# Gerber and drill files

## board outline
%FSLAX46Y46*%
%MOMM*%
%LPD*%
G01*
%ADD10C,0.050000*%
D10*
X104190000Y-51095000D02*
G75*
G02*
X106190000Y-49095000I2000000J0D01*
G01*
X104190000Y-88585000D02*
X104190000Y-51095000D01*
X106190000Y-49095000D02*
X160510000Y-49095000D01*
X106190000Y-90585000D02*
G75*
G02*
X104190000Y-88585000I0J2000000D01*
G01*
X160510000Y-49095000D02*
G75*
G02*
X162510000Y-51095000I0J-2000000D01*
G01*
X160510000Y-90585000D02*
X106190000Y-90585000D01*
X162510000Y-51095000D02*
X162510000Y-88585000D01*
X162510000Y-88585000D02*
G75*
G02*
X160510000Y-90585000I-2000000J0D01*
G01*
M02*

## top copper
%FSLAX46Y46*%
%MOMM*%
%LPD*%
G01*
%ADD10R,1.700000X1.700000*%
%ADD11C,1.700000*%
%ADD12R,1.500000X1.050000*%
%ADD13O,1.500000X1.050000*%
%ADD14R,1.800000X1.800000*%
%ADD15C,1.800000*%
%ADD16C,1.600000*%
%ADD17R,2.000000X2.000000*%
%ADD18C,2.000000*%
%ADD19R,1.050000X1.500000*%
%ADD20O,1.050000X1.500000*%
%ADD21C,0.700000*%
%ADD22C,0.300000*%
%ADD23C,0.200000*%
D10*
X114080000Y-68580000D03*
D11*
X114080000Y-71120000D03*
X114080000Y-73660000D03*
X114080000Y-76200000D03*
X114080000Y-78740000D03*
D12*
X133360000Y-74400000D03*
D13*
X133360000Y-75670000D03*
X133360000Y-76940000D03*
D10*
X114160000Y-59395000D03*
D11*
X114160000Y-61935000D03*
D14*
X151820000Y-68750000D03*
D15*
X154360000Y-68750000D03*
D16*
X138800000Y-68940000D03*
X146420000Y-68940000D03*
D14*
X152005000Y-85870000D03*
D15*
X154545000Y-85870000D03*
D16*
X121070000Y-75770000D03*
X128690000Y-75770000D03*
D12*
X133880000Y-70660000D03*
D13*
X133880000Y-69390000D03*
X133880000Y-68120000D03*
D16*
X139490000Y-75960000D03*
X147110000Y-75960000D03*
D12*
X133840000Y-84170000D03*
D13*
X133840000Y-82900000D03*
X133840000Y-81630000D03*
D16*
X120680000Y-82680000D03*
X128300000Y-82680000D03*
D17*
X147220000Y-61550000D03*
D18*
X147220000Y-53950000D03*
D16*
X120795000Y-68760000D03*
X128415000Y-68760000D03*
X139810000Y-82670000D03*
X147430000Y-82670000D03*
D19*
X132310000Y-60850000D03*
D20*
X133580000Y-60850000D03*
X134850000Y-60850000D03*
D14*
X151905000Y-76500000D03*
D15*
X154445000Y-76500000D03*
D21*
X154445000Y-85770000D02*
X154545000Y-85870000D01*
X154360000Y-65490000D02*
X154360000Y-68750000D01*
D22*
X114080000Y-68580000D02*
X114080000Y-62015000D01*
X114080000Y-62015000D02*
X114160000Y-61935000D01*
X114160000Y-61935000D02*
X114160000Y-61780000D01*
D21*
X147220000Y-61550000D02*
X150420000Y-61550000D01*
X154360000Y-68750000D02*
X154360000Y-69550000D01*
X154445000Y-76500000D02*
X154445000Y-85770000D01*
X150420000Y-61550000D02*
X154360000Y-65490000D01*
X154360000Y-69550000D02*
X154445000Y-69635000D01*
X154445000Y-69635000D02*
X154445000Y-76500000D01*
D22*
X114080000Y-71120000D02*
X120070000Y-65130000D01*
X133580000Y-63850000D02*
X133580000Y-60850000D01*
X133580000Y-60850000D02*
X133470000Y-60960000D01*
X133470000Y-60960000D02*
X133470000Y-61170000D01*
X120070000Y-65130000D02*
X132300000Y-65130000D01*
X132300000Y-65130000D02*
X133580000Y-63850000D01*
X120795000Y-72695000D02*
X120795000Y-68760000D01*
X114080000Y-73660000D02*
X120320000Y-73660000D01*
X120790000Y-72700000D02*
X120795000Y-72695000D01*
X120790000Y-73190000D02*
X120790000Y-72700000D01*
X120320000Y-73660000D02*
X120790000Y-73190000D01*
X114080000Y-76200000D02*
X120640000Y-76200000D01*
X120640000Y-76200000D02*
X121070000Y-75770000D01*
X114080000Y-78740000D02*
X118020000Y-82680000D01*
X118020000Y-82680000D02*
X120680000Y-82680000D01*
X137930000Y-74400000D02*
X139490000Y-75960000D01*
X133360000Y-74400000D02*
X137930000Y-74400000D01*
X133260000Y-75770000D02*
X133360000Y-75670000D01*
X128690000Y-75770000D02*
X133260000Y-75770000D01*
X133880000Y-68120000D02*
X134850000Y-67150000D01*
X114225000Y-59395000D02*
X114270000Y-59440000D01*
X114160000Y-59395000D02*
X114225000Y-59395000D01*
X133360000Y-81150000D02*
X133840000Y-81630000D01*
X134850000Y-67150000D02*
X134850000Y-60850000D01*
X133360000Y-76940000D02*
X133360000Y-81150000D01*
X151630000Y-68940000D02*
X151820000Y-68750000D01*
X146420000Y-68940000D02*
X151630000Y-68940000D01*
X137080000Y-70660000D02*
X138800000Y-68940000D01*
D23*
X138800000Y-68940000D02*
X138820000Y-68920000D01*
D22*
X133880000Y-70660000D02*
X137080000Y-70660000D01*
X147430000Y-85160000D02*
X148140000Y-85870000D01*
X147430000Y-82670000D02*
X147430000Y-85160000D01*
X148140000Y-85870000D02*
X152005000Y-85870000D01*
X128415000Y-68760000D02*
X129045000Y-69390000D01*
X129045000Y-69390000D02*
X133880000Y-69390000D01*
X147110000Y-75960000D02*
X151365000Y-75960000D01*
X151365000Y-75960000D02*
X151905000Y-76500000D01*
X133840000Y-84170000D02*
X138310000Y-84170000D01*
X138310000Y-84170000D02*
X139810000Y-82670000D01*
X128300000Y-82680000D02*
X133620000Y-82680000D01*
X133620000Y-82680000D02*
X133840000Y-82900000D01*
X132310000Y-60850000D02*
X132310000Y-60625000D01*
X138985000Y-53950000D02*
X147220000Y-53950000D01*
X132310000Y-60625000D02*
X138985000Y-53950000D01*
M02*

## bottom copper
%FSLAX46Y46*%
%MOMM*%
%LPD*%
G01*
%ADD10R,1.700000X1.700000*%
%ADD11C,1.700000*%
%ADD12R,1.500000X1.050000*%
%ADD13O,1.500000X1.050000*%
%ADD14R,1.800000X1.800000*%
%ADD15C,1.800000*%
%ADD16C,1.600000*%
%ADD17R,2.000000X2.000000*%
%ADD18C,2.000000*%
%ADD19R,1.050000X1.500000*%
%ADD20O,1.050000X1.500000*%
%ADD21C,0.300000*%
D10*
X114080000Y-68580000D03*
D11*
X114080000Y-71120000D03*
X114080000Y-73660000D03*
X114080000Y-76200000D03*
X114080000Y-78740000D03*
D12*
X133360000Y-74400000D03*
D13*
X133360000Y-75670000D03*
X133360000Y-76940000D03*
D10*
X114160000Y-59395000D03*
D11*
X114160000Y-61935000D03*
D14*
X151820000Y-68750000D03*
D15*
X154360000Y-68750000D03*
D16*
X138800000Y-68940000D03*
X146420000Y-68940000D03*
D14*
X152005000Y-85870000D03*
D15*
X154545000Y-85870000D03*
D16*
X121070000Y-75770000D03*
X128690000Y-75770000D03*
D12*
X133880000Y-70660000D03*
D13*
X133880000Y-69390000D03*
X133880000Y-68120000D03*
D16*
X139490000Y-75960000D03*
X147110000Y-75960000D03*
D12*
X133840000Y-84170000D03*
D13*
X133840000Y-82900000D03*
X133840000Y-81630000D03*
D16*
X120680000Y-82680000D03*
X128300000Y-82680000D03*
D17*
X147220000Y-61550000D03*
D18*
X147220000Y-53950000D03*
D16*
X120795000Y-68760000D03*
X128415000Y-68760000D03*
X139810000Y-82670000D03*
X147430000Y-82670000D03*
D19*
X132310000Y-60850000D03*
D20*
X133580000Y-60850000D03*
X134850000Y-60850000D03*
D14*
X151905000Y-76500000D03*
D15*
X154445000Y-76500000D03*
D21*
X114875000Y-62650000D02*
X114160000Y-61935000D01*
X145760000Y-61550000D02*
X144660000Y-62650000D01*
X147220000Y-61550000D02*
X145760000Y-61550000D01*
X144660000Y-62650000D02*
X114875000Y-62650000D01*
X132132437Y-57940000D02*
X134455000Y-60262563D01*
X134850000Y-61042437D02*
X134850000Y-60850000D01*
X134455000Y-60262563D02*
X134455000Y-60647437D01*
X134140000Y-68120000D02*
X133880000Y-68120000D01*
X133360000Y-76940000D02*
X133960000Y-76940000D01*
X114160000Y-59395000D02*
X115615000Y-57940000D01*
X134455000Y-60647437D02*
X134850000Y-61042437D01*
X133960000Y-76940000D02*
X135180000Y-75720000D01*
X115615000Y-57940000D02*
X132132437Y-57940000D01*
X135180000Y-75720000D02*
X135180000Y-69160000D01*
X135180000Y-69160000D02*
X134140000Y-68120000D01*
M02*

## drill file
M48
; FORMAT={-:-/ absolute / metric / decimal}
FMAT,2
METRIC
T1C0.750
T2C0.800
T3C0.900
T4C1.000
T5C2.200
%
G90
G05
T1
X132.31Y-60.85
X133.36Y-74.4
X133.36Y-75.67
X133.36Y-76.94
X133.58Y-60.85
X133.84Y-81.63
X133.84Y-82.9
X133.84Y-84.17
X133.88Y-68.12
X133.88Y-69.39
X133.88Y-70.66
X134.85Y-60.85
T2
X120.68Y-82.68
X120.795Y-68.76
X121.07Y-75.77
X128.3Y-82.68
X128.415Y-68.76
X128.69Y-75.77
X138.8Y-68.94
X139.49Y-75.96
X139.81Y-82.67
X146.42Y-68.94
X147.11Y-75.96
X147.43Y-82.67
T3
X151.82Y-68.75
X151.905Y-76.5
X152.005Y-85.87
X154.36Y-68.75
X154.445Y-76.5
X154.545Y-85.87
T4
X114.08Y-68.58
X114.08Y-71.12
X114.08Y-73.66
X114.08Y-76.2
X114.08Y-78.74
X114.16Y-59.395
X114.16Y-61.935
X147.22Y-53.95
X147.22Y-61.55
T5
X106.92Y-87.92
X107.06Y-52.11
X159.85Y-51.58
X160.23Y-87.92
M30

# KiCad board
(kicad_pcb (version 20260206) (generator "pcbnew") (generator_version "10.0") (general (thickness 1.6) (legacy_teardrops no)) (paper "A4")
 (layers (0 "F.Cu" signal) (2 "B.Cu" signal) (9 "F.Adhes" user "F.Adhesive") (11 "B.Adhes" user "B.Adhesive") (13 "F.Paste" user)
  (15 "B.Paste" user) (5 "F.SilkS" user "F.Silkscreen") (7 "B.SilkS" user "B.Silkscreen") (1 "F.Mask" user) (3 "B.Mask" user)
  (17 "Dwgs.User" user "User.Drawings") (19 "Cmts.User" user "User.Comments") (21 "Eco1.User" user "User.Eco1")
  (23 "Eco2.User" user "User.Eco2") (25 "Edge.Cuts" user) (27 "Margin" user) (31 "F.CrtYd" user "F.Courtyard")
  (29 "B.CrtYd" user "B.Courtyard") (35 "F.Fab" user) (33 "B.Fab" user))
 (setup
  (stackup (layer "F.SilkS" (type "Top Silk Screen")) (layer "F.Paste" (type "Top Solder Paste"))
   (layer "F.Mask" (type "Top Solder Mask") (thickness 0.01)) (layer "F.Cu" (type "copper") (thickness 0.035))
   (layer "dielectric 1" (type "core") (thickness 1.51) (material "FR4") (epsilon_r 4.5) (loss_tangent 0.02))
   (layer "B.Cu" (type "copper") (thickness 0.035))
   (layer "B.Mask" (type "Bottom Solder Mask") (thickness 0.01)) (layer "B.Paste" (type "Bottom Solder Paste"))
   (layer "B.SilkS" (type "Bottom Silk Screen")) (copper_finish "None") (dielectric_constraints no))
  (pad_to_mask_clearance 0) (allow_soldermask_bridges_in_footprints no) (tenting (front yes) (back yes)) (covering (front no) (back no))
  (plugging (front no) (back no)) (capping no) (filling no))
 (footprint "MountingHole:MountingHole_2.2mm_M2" (layer "F.Cu") (at 106.92 87.92)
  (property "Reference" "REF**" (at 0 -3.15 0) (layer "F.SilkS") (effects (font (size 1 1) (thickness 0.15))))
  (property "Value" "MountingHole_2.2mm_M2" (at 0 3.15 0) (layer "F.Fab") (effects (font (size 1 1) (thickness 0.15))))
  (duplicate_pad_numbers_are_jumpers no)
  (pad "" np_thru_hole circle (at 0 0) (size 2.2 2.2) (drill 2.2) (layers "*.Cu" "*.Mask")))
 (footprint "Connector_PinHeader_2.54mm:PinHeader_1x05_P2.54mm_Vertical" (layer "F.Cu") (at 114.08 68.58)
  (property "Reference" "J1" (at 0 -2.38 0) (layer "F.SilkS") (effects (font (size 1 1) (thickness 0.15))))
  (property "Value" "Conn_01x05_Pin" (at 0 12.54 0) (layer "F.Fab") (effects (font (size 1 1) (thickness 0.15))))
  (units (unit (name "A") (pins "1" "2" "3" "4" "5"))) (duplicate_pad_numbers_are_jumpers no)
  (pad "1" thru_hole rect (at 0 0) (size 1.7 1.7) (drill 1) (layers "*.Cu" "*.Mask") (remove_unused_layers no) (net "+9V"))
  (pad "2" thru_hole circle (at 0 2.54) (size 1.7 1.7) (drill 1) (layers "*.Cu" "*.Mask") (remove_unused_layers no) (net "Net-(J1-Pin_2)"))
  (pad "3" thru_hole circle (at 0 5.08) (size 1.7 1.7) (drill 1) (layers "*.Cu" "*.Mask") (remove_unused_layers no) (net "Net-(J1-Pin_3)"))
  (pad "4" thru_hole circle (at 0 7.62) (size 1.7 1.7) (drill 1) (layers "*.Cu" "*.Mask") (remove_unused_layers no) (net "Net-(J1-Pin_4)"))
  (pad "5" thru_hole circle (at 0 10.16) (size 1.7 1.7) (drill 1) (layers "*.Cu" "*.Mask") (remove_unused_layers no) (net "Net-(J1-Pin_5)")))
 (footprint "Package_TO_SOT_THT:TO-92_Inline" (layer "F.Cu") (at 133.36 74.4 -90)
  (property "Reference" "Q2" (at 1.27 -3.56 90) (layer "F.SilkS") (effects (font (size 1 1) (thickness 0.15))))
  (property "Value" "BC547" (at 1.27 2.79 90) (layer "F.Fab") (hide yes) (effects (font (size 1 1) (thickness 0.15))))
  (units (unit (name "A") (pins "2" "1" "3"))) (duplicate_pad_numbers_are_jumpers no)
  (pad "1" thru_hole rect (at 0 0 270) (size 1.05 1.5) (drill 0.75) (layers "*.Cu" "*.Mask") (remove_unused_layers no) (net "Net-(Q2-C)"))
  (pad "2" thru_hole oval (at 1.27 0 270) (size 1.05 1.5) (drill 0.75) (layers "*.Cu" "*.Mask") (remove_unused_layers no) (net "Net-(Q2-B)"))
  (pad "3" thru_hole oval (at 2.54 0 270) (size 1.05 1.5) (drill 0.75) (layers "*.Cu" "*.Mask") (remove_unused_layers no) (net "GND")))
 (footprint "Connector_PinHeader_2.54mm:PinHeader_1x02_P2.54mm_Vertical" (layer "F.Cu") (at 114.16 59.395)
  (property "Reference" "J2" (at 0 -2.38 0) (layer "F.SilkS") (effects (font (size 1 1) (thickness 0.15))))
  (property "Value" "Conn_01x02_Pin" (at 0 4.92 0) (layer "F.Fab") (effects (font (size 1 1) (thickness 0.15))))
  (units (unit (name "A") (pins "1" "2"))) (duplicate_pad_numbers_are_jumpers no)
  (pad "1" thru_hole rect (at 0 0) (size 1.7 1.7) (drill 1) (layers "*.Cu" "*.Mask") (remove_unused_layers no) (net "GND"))
  (pad "2" thru_hole circle (at 0 2.54) (size 1.7 1.7) (drill 1) (layers "*.Cu" "*.Mask") (remove_unused_layers no) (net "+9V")))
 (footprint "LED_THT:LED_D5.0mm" (layer "F.Cu") (at 151.82 68.75)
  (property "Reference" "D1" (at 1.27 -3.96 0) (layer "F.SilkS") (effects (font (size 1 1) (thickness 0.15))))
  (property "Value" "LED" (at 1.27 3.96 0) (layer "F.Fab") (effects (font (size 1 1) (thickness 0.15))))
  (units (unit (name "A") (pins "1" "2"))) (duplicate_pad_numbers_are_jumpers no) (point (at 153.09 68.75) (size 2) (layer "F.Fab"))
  (pad "1" thru_hole rect (at 0 0) (size 1.8 1.8) (drill 0.9) (layers "*.Cu" "*.Mask") (remove_unused_layers no) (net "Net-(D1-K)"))
  (pad "2" thru_hole circle (at 2.54 0) (size 1.8 1.8) (drill 0.9) (layers "*.Cu" "*.Mask") (remove_unused_layers no) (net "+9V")))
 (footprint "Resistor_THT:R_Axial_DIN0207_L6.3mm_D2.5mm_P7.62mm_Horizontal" (layer "F.Cu") (at 138.8 68.94)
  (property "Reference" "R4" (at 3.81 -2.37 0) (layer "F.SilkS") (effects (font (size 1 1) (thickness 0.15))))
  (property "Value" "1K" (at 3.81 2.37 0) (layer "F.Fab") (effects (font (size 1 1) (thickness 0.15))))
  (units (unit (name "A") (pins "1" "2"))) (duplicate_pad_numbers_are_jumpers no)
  (pad "1" thru_hole circle (at 0 0) (size 1.6 1.6) (drill 0.8) (layers "*.Cu" "*.Mask") (remove_unused_layers no) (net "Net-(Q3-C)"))
  (pad "2" thru_hole circle (at 7.62 0) (size 1.6 1.6) (drill 0.8) (layers "*.Cu" "*.Mask") (remove_unused_layers no) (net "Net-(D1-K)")))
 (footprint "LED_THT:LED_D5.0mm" (layer "F.Cu") (at 152.005 85.87)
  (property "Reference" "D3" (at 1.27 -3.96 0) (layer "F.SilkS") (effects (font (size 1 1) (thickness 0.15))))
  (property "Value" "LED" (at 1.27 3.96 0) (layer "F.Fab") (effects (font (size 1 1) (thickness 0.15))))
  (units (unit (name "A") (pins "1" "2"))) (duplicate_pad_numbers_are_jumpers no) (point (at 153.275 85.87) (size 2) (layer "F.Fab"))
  (pad "1" thru_hole rect (at 0 0) (size 1.8 1.8) (drill 0.9) (layers "*.Cu" "*.Mask") (remove_unused_layers no) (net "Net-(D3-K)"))
  (pad "2" thru_hole circle (at 2.54 0) (size 1.8 1.8) (drill 0.9) (layers "*.Cu" "*.Mask") (remove_unused_layers no) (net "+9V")))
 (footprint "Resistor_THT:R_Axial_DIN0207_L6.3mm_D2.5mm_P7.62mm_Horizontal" (layer "F.Cu") (at 121.07 75.77)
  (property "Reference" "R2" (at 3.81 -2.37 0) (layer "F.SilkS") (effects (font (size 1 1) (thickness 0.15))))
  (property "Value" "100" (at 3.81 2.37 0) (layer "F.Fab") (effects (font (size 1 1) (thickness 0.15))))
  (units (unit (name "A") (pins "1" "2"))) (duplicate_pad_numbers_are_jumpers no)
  (pad "1" thru_hole circle (at 0 0) (size 1.6 1.6) (drill 0.8) (layers "*.Cu" "*.Mask") (remove_unused_layers no) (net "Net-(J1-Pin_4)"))
  (pad "2" thru_hole circle (at 7.62 0) (size 1.6 1.6) (drill 0.8) (layers "*.Cu" "*.Mask") (remove_unused_layers no) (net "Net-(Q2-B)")))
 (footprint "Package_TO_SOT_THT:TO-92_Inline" (layer "F.Cu") (at 133.88 70.66 90)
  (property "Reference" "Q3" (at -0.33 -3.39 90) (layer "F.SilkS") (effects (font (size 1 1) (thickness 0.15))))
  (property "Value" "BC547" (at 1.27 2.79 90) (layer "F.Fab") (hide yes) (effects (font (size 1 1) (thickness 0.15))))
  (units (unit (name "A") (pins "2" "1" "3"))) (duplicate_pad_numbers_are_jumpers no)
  (pad "1" thru_hole rect (at 0 0 90) (size 1.05 1.5) (drill 0.75) (layers "*.Cu" "*.Mask") (remove_unused_layers no) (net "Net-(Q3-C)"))
  (pad "2" thru_hole oval (at 1.27 0 90) (size 1.05 1.5) (drill 0.75) (layers "*.Cu" "*.Mask") (remove_unused_layers no) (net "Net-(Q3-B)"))
  (pad "3" thru_hole oval (at 2.54 0 90) (size 1.05 1.5) (drill 0.75) (layers "*.Cu" "*.Mask") (remove_unused_layers no) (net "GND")))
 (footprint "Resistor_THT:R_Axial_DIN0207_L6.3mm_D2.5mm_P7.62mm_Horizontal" (layer "F.Cu") (at 139.49 75.96)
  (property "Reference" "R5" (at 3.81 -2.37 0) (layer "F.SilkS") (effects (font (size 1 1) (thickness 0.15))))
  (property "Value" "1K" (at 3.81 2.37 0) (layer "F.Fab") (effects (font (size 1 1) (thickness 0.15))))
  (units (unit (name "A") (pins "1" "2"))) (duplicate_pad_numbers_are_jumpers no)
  (pad "1" thru_hole circle (at 0 0) (size 1.6 1.6) (drill 0.8) (layers "*.Cu" "*.Mask") (remove_unused_layers no) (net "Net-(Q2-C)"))
  (pad "2" thru_hole circle (at 7.62 0) (size 1.6 1.6) (drill 0.8) (layers "*.Cu" "*.Mask") (remove_unused_layers no) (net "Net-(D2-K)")))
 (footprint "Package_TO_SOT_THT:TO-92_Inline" (layer "F.Cu") (at 133.84 84.17 90)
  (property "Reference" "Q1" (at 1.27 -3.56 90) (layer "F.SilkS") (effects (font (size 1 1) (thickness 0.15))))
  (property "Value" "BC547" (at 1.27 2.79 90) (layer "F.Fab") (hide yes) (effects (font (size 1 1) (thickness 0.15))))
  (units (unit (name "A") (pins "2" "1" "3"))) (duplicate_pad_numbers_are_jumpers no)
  (pad "1" thru_hole rect (at 0 0 90) (size 1.05 1.5) (drill 0.75) (layers "*.Cu" "*.Mask") (remove_unused_layers no) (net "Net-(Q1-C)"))
  (pad "2" thru_hole oval (at 1.27 0 90) (size 1.05 1.5) (drill 0.75) (layers "*.Cu" "*.Mask") (remove_unused_layers no) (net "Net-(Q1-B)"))
  (pad "3" thru_hole oval (at 2.54 0 90) (size 1.05 1.5) (drill 0.75) (layers "*.Cu" "*.Mask") (remove_unused_layers no) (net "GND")))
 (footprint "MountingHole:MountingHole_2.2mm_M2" (layer "F.Cu") (at 160.23 87.92)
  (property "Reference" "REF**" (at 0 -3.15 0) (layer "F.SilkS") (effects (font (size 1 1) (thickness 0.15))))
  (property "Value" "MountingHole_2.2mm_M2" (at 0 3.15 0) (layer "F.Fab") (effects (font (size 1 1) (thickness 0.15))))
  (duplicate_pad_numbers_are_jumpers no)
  (pad "" np_thru_hole circle (at 0 0) (size 2.2 2.2) (drill 2.2) (layers "*.Cu" "*.Mask")))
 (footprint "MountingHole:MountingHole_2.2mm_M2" (layer "F.Cu") (at 159.85 51.58)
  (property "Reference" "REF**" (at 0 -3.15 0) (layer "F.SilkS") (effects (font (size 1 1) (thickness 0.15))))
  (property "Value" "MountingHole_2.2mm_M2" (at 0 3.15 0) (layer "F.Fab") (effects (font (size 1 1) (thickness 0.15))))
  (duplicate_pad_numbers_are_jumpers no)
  (pad "" np_thru_hole circle (at 0 0) (size 2.2 2.2) (drill 2.2) (layers "*.Cu" "*.Mask")))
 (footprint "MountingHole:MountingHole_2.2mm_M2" (layer "F.Cu") (at 107.06 52.11)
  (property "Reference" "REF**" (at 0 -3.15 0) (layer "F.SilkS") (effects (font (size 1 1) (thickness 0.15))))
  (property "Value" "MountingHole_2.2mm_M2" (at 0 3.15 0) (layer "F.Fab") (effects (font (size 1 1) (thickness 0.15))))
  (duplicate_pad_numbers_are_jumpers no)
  (pad "" np_thru_hole circle (at 0 0) (size 2.2 2.2) (drill 2.2) (layers "*.Cu" "*.Mask")))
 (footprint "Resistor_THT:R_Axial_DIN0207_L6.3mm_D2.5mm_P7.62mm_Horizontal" (layer "F.Cu") (at 120.68 82.68)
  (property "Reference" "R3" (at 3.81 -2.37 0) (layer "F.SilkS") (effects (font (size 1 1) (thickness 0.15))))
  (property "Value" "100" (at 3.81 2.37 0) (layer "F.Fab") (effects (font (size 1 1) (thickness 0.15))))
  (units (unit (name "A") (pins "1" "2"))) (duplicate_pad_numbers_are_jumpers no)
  (pad "1" thru_hole circle (at 0 0) (size 1.6 1.6) (drill 0.8) (layers "*.Cu" "*.Mask") (remove_unused_layers no) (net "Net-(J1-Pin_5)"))
  (pad "2" thru_hole circle (at 7.62 0) (size 1.6 1.6) (drill 0.8) (layers "*.Cu" "*.Mask") (remove_unused_layers no) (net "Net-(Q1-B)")))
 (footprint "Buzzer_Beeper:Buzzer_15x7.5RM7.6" (layer "F.Cu") (at 147.22 61.55 90)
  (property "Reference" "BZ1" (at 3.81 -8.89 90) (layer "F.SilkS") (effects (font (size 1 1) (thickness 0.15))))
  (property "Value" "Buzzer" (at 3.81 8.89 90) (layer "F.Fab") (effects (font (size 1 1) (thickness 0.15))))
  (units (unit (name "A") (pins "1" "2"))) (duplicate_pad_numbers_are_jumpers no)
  (pad "1" thru_hole rect (at 0 0 90) (size 2 2) (drill 1) (layers "*.Cu" "*.Mask") (remove_unused_layers no) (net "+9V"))
  (pad "2" thru_hole circle (at 7.6 0 90) (size 2 2) (drill 1) (layers "*.Cu" "*.Mask") (remove_unused_layers no) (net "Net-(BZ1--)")))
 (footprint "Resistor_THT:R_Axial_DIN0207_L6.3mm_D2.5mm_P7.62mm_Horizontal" (layer "F.Cu") (at 120.795 68.76)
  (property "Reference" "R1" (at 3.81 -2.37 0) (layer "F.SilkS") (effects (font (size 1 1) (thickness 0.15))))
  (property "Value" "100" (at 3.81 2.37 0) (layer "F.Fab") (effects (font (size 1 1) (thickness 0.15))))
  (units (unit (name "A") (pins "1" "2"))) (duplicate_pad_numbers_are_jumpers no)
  (pad "1" thru_hole circle (at 0 0) (size 1.6 1.6) (drill 0.8) (layers "*.Cu" "*.Mask") (remove_unused_layers no) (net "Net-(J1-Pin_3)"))
  (pad "2" thru_hole circle (at 7.62 0) (size 1.6 1.6) (drill 0.8) (layers "*.Cu" "*.Mask") (remove_unused_layers no) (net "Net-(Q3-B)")))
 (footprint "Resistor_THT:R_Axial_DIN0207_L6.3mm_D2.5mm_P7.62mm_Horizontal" (layer "F.Cu") (at 139.81 82.67)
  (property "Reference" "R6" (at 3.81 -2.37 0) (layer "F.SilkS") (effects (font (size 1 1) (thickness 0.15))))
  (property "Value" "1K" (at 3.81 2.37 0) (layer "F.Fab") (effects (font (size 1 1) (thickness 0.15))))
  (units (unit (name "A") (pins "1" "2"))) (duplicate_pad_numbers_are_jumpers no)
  (pad "1" thru_hole circle (at 0 0) (size 1.6 1.6) (drill 0.8) (layers "*.Cu" "*.Mask") (remove_unused_layers no) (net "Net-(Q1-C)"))
  (pad "2" thru_hole circle (at 7.62 0) (size 1.6 1.6) (drill 0.8) (layers "*.Cu" "*.Mask") (remove_unused_layers no) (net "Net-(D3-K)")))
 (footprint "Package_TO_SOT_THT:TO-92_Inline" (layer "F.Cu") (at 132.31 60.85)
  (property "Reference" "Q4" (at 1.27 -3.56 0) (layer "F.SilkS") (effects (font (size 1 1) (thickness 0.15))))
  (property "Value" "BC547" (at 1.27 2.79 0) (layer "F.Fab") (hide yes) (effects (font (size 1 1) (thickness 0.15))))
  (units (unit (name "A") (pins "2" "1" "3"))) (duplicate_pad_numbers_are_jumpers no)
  (pad "1" thru_hole rect (at 0 0) (size 1.05 1.5) (drill 0.75) (layers "*.Cu" "*.Mask") (remove_unused_layers no) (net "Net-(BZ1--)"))
  (pad "2" thru_hole oval (at 1.27 0) (size 1.05 1.5) (drill 0.75) (layers "*.Cu" "*.Mask") (remove_unused_layers no) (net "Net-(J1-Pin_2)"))
  (pad "3" thru_hole oval (at 2.54 0) (size 1.05 1.5) (drill 0.75) (layers "*.Cu" "*.Mask") (remove_unused_layers no) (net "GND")))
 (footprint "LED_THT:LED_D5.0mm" (layer "F.Cu") (at 151.905 76.5)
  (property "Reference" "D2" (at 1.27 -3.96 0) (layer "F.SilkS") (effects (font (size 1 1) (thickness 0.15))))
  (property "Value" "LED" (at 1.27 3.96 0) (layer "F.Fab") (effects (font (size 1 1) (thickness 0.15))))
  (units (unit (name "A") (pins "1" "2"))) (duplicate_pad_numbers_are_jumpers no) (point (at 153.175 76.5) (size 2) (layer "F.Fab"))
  (pad "1" thru_hole rect (at 0 0) (size 1.8 1.8) (drill 0.9) (layers "*.Cu" "*.Mask") (remove_unused_layers no) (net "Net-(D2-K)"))
  (pad "2" thru_hole circle (at 2.54 0) (size 1.8 1.8) (drill 0.9) (layers "*.Cu" "*.Mask") (remove_unused_layers no) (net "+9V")))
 (gr_arc (start 104.19 51.095) (mid 104.775786 49.680786) (end 106.19 49.095) (stroke (width 0.05) (type default)) (layer "Edge.Cuts"))
 (gr_line (start 104.19 88.585) (end 104.19 51.095) (stroke (width 0.05) (type default)) (layer "Edge.Cuts"))
 (gr_line (start 106.19 49.095) (end 160.51 49.095) (stroke (width 0.05) (type default)) (layer "Edge.Cuts"))
 (gr_arc (start 106.19 90.585) (mid 104.775786 89.999214) (end 104.19 88.585) (stroke (width 0.05) (type default)) (layer "Edge.Cuts"))
 (gr_arc (start 160.51 49.095) (mid 161.924214 49.680786) (end 162.51 51.095) (stroke (width 0.05) (type default)) (layer "Edge.Cuts"))
 (gr_line (start 160.51 90.585) (end 106.19 90.585) (stroke (width 0.05) (type default)) (layer "Edge.Cuts"))
 (gr_line (start 162.51 51.095) (end 162.51 88.585) (stroke (width 0.05) (type default)) (layer "Edge.Cuts"))
 (gr_arc (start 162.51 88.585) (mid 161.924214 89.999214) (end 160.51 90.585) (stroke (width 0.05) (type default)) (layer "Edge.Cuts"))
 (segment (start 154.445 85.77) (end 154.545 85.87) (width 0.7) (layer "F.Cu") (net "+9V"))
 (segment (start 154.36 65.49) (end 154.36 68.75) (width 0.7) (layer "F.Cu") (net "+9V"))
 (segment (start 114.08 68.58) (end 114.08 62.015) (width 0.3) (layer "F.Cu") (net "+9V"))
 (segment (start 114.08 62.015) (end 114.16 61.935) (width 0.3) (layer "F.Cu") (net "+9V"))
 (segment (start 114.16 61.935) (end 114.16 61.78) (width 0.3) (layer "F.Cu") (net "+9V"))
 (segment (start 147.22 61.55) (end 150.42 61.55) (width 0.7) (layer "F.Cu") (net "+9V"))
 (segment (start 154.36 68.75) (end 154.36 69.55) (width 0.7) (layer "F.Cu") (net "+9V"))
 (segment (start 154.445 76.5) (end 154.445 85.77) (width 0.7) (layer "F.Cu") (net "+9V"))
 (segment (start 150.42 61.55) (end 154.36 65.49) (width 0.7) (layer "F.Cu") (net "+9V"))
 (segment (start 154.36 69.55) (end 154.445 69.635) (width 0.7) (layer "F.Cu") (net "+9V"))
 (segment (start 154.445 69.635) (end 154.445 76.5) (width 0.7) (layer "F.Cu") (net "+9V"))
 (segment (start 114.875 62.65) (end 114.16 61.935) (width 0.3) (layer "B.Cu") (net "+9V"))
 (segment (start 145.76 61.55) (end 144.66 62.65) (width 0.3) (layer "B.Cu") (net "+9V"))
 (segment (start 147.22 61.55) (end 145.76 61.55) (width 0.3) (layer "B.Cu") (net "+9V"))
 (segment (start 144.66 62.65) (end 114.875 62.65) (width 0.3) (layer "B.Cu") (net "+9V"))
 (segment (start 114.08 71.12) (end 120.07 65.13) (width 0.3) (layer "F.Cu") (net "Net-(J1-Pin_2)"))
 (segment (start 133.58 63.85) (end 133.58 60.85) (width 0.3) (layer "F.Cu") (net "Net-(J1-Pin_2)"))
 (segment (start 133.58 60.85) (end 133.47 60.96) (width 0.3) (layer "F.Cu") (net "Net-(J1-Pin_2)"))
 (segment (start 133.47 60.96) (end 133.47 61.17) (width 0.3) (layer "F.Cu") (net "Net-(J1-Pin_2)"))
 (segment (start 120.07 65.13) (end 132.3 65.13) (width 0.3) (layer "F.Cu") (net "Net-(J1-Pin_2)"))
 (segment (start 132.3 65.13) (end 133.58 63.85) (width 0.3) (layer "F.Cu") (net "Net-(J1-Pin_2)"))
 (segment (start 120.795 72.695) (end 120.795 68.76) (width 0.3) (layer "F.Cu") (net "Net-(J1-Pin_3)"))
 (segment (start 114.08 73.66) (end 120.32 73.66) (width 0.3) (layer "F.Cu") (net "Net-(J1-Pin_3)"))
 (segment (start 120.79 72.7) (end 120.795 72.695) (width 0.3) (layer "F.Cu") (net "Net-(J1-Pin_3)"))
 (segment (start 120.79 73.19) (end 120.79 72.7) (width 0.3) (layer "F.Cu") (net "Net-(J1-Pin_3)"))
 (segment (start 120.32 73.66) (end 120.79 73.19) (width 0.3) (layer "F.Cu") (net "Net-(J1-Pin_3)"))
 (segment (start 114.08 76.2) (end 120.64 76.2) (width 0.3) (layer "F.Cu") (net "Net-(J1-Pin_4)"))
 (segment (start 120.64 76.2) (end 121.07 75.77) (width 0.3) (layer "F.Cu") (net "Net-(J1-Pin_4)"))
 (segment (start 114.08 78.74) (end 118.02 82.68) (width 0.3) (layer "F.Cu") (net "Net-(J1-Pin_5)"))
 (segment (start 118.02 82.68) (end 120.68 82.68) (width 0.3) (layer "F.Cu") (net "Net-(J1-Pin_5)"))
 (segment (start 137.93 74.4) (end 139.49 75.96) (width 0.3) (layer "F.Cu") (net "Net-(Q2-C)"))
 (segment (start 133.36 74.4) (end 137.93 74.4) (width 0.3) (layer "F.Cu") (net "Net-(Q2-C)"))
 (segment (start 133.26 75.77) (end 133.36 75.67) (width 0.3) (layer "F.Cu") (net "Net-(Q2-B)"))
 (segment (start 128.69 75.77) (end 133.26 75.77) (width 0.3) (layer "F.Cu") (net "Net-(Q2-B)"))
 (segment (start 133.88 68.12) (end 134.85 67.15) (width 0.3) (layer "F.Cu") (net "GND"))
 (segment (start 114.225 59.395) (end 114.27 59.44) (width 0.3) (layer "F.Cu") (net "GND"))
 (segment (start 114.16 59.395) (end 114.225 59.395) (width 0.3) (layer "F.Cu") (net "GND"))
 (segment (start 133.36 81.15) (end 133.84 81.63) (width 0.3) (layer "F.Cu") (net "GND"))
 (segment (start 134.85 67.15) (end 134.85 60.85) (width 0.3) (layer "F.Cu") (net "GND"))
 (segment (start 133.36 76.94) (end 133.36 81.15) (width 0.3) (layer "F.Cu") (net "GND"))
 (segment (start 132.132437 57.94) (end 134.455 60.262563) (width 0.3) (layer "B.Cu") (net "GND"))
 (segment (start 134.85 61.042437) (end 134.85 60.85) (width 0.3) (layer "B.Cu") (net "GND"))
 (segment (start 134.455 60.262563) (end 134.455 60.647437) (width 0.3) (layer "B.Cu") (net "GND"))
 (segment (start 134.14 68.12) (end 133.88 68.12) (width 0.3) (layer "B.Cu") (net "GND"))
 (segment (start 133.36 76.94) (end 133.96 76.94) (width 0.3) (layer "B.Cu") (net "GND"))
 (segment (start 114.16 59.395) (end 115.615 57.94) (width 0.3) (layer "B.Cu") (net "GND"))
 (segment (start 134.455 60.647437) (end 134.85 61.042437) (width 0.3) (layer "B.Cu") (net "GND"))
 (segment (start 133.96 76.94) (end 135.18 75.72) (width 0.3) (layer "B.Cu") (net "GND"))
 (segment (start 115.615 57.94) (end 132.132437 57.94) (width 0.3) (layer "B.Cu") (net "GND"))
 (segment (start 135.18 75.72) (end 135.18 69.16) (width 0.3) (layer "B.Cu") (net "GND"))
 (segment (start 135.18 69.16) (end 134.14 68.12) (width 0.3) (layer "B.Cu") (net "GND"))
 (segment (start 151.63 68.94) (end 151.82 68.75) (width 0.3) (layer "F.Cu") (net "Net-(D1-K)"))
 (segment (start 146.42 68.94) (end 151.63 68.94) (width 0.3) (layer "F.Cu") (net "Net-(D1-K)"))
 (segment (start 137.08 70.66) (end 138.8 68.94) (width 0.3) (layer "F.Cu") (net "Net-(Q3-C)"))
 (segment (start 138.8 68.94) (end 138.82 68.92) (width 0.2) (layer "F.Cu") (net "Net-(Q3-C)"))
 (segment (start 133.88 70.66) (end 137.08 70.66) (width 0.3) (layer "F.Cu") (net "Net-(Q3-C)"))
 (segment (start 147.43 85.16) (end 148.14 85.87) (width 0.3) (layer "F.Cu") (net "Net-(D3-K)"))
 (segment (start 147.43 82.67) (end 147.43 85.16) (width 0.3) (layer "F.Cu") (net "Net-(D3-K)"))
 (segment (start 148.14 85.87) (end 152.005 85.87) (width 0.3) (layer "F.Cu") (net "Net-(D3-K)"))
 (segment (start 128.415 68.76) (end 129.045 69.39) (width 0.3) (layer "F.Cu") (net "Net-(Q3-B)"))
 (segment (start 129.045 69.39) (end 133.88 69.39) (width 0.3) (layer "F.Cu") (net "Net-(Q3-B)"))
 (segment (start 147.11 75.96) (end 151.365 75.96) (width 0.3) (layer "F.Cu") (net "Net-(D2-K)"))
 (segment (start 151.365 75.96) (end 151.905 76.5) (width 0.3) (layer "F.Cu") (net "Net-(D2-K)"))
 (segment (start 133.84 84.17) (end 138.31 84.17) (width 0.3) (layer "F.Cu") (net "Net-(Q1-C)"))
 (segment (start 138.31 84.17) (end 139.81 82.67) (width 0.3) (layer "F.Cu") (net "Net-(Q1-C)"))
 (segment (start 128.3 82.68) (end 133.62 82.68) (width 0.3) (layer "F.Cu") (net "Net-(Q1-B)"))
 (segment (start 133.62 82.68) (end 133.84 82.9) (width 0.3) (layer "F.Cu") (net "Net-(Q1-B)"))
 (segment (start 132.31 60.85) (end 132.31 60.625) (width 0.3) (layer "F.Cu") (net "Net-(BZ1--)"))
 (segment (start 138.985 53.95) (end 147.22 53.95) (width 0.3) (layer "F.Cu") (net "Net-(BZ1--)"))
 (segment (start 132.31 60.625) (end 138.985 53.95) (width 0.3) (layer "F.Cu") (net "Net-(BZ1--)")))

